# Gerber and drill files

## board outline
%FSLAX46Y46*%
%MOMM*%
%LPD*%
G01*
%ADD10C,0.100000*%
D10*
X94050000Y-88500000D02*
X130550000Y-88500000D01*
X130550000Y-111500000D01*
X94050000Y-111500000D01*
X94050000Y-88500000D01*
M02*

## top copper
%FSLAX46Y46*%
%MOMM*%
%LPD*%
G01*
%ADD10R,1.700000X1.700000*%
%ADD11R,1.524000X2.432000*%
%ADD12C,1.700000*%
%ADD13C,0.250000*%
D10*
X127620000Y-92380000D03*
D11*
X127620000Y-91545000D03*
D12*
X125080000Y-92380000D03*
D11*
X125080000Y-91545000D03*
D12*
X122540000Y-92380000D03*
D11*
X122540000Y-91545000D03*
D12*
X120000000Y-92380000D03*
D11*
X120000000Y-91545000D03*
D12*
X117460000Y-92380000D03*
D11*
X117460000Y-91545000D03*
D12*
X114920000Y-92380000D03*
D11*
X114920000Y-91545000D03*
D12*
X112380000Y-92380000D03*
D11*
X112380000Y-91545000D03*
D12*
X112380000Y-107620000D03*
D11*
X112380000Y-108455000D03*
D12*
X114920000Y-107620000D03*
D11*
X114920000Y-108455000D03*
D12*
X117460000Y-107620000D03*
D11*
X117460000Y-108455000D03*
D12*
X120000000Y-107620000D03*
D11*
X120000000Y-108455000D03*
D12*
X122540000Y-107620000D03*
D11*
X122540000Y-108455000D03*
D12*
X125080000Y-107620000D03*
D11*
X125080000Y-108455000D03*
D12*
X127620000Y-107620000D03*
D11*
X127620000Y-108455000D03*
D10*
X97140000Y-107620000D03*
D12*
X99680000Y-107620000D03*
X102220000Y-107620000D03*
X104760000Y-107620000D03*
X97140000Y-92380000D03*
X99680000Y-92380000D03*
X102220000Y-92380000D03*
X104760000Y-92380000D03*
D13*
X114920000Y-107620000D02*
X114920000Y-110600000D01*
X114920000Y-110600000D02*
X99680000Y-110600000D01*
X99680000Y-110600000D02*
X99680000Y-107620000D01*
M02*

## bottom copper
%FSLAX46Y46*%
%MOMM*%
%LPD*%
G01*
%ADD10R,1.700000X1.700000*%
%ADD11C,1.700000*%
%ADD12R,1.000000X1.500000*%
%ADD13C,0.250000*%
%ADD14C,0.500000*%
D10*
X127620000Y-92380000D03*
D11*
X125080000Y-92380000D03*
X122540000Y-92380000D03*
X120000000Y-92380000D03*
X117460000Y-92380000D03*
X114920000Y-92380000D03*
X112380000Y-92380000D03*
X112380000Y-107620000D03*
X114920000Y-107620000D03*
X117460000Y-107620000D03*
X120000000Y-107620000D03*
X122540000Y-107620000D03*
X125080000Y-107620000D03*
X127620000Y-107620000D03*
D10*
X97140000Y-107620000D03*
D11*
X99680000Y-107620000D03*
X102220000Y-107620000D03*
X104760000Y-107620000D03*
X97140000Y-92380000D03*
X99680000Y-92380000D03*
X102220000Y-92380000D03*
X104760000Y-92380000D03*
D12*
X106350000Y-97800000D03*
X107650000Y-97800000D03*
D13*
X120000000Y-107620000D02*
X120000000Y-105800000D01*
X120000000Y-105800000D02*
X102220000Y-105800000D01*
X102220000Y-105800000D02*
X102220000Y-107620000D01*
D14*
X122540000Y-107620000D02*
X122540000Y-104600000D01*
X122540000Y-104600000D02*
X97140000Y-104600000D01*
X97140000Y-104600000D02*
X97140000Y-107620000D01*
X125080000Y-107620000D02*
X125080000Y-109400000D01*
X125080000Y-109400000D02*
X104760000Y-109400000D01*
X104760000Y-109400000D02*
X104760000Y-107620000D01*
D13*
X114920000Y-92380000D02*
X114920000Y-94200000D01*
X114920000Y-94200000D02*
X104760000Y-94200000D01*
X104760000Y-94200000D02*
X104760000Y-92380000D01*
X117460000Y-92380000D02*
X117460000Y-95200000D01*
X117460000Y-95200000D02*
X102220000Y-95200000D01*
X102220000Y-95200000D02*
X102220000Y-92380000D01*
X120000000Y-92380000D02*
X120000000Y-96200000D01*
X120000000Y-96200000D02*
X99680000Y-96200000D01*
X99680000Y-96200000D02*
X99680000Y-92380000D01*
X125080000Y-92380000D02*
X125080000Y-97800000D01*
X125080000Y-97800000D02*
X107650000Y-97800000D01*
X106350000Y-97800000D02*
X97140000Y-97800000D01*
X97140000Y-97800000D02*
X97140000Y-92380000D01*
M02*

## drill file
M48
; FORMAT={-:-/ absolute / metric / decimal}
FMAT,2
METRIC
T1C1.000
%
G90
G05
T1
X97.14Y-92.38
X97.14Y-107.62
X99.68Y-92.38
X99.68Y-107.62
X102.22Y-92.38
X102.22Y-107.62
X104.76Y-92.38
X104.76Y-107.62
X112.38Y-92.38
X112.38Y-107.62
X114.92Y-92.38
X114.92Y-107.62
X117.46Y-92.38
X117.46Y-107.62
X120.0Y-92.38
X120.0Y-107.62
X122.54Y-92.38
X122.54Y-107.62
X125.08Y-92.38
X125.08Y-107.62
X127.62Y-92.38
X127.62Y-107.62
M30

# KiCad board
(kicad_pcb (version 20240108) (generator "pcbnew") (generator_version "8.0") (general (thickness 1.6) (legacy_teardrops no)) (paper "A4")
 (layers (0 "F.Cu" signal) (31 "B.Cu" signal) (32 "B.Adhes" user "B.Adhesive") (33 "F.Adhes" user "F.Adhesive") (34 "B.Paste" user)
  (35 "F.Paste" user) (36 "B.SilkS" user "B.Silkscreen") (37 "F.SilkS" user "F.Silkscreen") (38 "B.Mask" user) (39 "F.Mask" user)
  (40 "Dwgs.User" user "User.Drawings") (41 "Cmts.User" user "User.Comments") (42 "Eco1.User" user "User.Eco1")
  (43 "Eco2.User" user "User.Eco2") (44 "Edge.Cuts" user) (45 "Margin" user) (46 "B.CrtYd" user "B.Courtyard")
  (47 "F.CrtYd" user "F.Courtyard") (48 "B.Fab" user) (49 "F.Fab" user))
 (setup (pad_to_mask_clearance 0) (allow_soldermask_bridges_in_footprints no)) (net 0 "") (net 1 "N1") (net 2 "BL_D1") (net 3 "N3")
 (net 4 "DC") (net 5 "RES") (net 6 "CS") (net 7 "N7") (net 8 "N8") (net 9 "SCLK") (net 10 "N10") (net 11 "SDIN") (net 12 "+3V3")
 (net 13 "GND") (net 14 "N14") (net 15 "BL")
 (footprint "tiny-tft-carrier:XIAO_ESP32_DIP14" (layer "F.Cu") (at 120 100)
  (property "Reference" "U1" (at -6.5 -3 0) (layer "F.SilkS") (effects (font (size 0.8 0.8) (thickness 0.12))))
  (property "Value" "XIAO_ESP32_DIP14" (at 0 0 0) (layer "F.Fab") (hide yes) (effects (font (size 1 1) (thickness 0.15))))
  (pad "1" thru_hole rect (at 7.62 -7.62) (size 1.7 1.7) (drill 1) (layers "*.Cu" "*.Mask") (remove_unused_layers no) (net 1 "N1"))
  (pad "1" smd rect (at 7.62 -8.455) (size 1.524 2.432) (layers "F.Cu" "F.Mask") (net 1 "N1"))
  (pad "2" thru_hole circle (at 5.08 -7.62) (size 1.7 1.7) (drill 1) (layers "*.Cu" "*.Mask") (remove_unused_layers no) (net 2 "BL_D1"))
  (pad "2" smd rect (at 5.08 -8.455) (size 1.524 2.432) (layers "F.Cu" "F.Mask") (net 2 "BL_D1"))
  (pad "3" thru_hole circle (at 2.54 -7.62) (size 1.7 1.7) (drill 1) (layers "*.Cu" "*.Mask") (remove_unused_layers no) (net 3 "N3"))
  (pad "3" smd rect (at 2.54 -8.455) (size 1.524 2.432) (layers "F.Cu" "F.Mask") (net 3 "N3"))
  (pad "4" thru_hole circle (at 0 -7.62) (size 1.7 1.7) (drill 1) (layers "*.Cu" "*.Mask") (remove_unused_layers no) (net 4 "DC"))
  (pad "4" smd rect (at 0 -8.455) (size 1.524 2.432) (layers "F.Cu" "F.Mask") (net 4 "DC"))
  (pad "5" thru_hole circle (at -2.54 -7.62) (size 1.7 1.7) (drill 1) (layers "*.Cu" "*.Mask") (remove_unused_layers no) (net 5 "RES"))
  (pad "5" smd rect (at -2.54 -8.455) (size 1.524 2.432) (layers "F.Cu" "F.Mask") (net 5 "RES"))
  (pad "6" thru_hole circle (at -5.08 -7.62) (size 1.7 1.7) (drill 1) (layers "*.Cu" "*.Mask") (remove_unused_layers no) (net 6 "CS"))
  (pad "6" smd rect (at -5.08 -8.455) (size 1.524 2.432) (layers "F.Cu" "F.Mask") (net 6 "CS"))
  (pad "7" thru_hole circle (at -7.62 -7.62) (size 1.7 1.7) (drill 1) (layers "*.Cu" "*.Mask") (remove_unused_layers no) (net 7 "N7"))
  (pad "7" smd rect (at -7.62 -8.455) (size 1.524 2.432) (layers "F.Cu" "F.Mask") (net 7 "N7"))
  (pad "8" thru_hole circle (at -7.62 7.62) (size 1.7 1.7) (drill 1) (layers "*.Cu" "*.Mask") (remove_unused_layers no) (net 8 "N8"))
  (pad "8" smd rect (at -7.62 8.455) (size 1.524 2.432) (layers "F.Cu" "F.Mask") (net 8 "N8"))
  (pad "9" thru_hole circle (at -5.08 7.62) (size 1.7 1.7) (drill 1) (layers "*.Cu" "*.Mask") (remove_unused_layers no) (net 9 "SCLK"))
  (pad "9" smd rect (at -5.08 8.455) (size 1.524 2.432) (layers "F.Cu" "F.Mask") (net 9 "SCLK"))
  (pad "10" thru_hole circle (at -2.54 7.62) (size 1.7 1.7) (drill 1) (layers "*.Cu" "*.Mask") (remove_unused_layers no) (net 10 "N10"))
  (pad "10" smd rect (at -2.54 8.455) (size 1.524 2.432) (layers "F.Cu" "F.Mask") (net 10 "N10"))
  (pad "11" thru_hole circle (at 0 7.62) (size 1.7 1.7) (drill 1) (layers "*.Cu" "*.Mask") (remove_unused_layers no) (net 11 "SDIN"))
  (pad "11" smd rect (at 0 8.455) (size 1.524 2.432) (layers "F.Cu" "F.Mask") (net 11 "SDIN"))
  (pad "12" thru_hole circle (at 2.54 7.62) (size 1.7 1.7) (drill 1) (layers "*.Cu" "*.Mask") (remove_unused_layers no) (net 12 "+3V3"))
  (pad "12" smd rect (at 2.54 8.455) (size 1.524 2.432) (layers "F.Cu" "F.Mask") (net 12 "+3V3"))
  (pad "13" thru_hole circle (at 5.08 7.62) (size 1.7 1.7) (drill 1) (layers "*.Cu" "*.Mask") (remove_unused_layers no) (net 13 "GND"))
  (pad "13" smd rect (at 5.08 8.455) (size 1.524 2.432) (layers "F.Cu" "F.Mask") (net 13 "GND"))
  (pad "14" thru_hole circle (at 7.62 7.62) (size 1.7 1.7) (drill 1) (layers "*.Cu" "*.Mask") (remove_unused_layers no) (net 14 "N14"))
  (pad "14" smd rect (at 7.62 8.455) (size 1.524 2.432) (layers "F.Cu" "F.Mask") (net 14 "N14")))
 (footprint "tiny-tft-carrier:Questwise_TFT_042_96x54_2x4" (layer "F.Cu") (at 100.95 100)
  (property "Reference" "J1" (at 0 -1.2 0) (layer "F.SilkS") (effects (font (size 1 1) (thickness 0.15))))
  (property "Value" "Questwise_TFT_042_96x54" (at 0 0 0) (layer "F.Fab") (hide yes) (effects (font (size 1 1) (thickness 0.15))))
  (pad "1" thru_hole rect (at -3.81 7.62) (size 1.7 1.7) (drill 1) (layers "*.Cu" "*.Mask") (remove_unused_layers no) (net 12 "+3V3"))
  (pad "2" thru_hole circle (at -1.27 7.62) (size 1.7 1.7) (drill 1) (layers "*.Cu" "*.Mask") (remove_unused_layers no) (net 9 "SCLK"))
  (pad "3" thru_hole circle (at 1.27 7.62) (size 1.7 1.7) (drill 1) (layers "*.Cu" "*.Mask") (remove_unused_layers no) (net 11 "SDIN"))
  (pad "4" thru_hole circle (at 3.81 7.62) (size 1.7 1.7) (drill 1) (layers "*.Cu" "*.Mask") (remove_unused_layers no) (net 13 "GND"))
  (pad "5" thru_hole circle (at -3.81 -7.62) (size 1.7 1.7) (drill 1) (layers "*.Cu" "*.Mask") (remove_unused_layers no) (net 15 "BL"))
  (pad "6" thru_hole circle (at -1.27 -7.62) (size 1.7 1.7) (drill 1) (layers "*.Cu" "*.Mask") (remove_unused_layers no) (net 4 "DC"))
  (pad "7" thru_hole circle (at 1.27 -7.62) (size 1.7 1.7) (drill 1) (layers "*.Cu" "*.Mask") (remove_unused_layers no) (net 5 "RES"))
  (pad "8" thru_hole circle (at 3.81 -7.62) (size 1.7 1.7) (drill 1) (layers "*.Cu" "*.Mask") (remove_unused_layers no) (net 6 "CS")))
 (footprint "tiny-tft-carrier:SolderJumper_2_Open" (layer "B.Cu") (at 107 97.8)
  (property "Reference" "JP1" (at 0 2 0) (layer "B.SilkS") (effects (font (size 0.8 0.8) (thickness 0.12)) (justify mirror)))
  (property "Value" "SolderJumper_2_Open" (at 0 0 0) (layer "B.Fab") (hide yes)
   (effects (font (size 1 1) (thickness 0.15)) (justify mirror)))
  (pad "1" smd rect (at -0.65 0) (size 1 1.5) (layers "B.Cu" "B.Mask") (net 15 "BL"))
  (pad "2" smd rect (at 0.65 0) (size 1 1.5) (layers "B.Cu" "B.Mask") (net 2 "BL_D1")))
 (gr_rect (start 94.05 88.5) (end 130.55 111.5) (stroke (width 0.1) (type default)) (fill no) (layer "Edge.Cuts"))
 (segment (start 120 107.62) (end 120 105.8) (width 0.25) (layer "B.Cu") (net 11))
 (segment (start 120 105.8) (end 102.22 105.8) (width 0.25) (layer "B.Cu") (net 11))
 (segment (start 102.22 105.8) (end 102.22 107.62) (width 0.25) (layer "B.Cu") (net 11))
 (segment (start 122.54 107.62) (end 122.54 104.6) (width 0.5) (layer "B.Cu") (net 12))
 (segment (start 122.54 104.6) (end 97.14 104.6) (width 0.5) (layer "B.Cu") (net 12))
 (segment (start 97.14 104.6) (end 97.14 107.62) (width 0.5) (layer "B.Cu") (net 12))
 (segment (start 125.08 107.62) (end 125.08 109.4) (width 0.5) (layer "B.Cu") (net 13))
 (segment (start 125.08 109.4) (end 104.76 109.4) (width 0.5) (layer "B.Cu") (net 13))
 (segment (start 104.76 109.4) (end 104.76 107.62) (width 0.5) (layer "B.Cu") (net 13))
 (segment (start 114.92 107.62) (end 114.92 110.6) (width 0.25) (layer "F.Cu") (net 9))
 (segment (start 114.92 110.6) (end 99.68 110.6) (width 0.25) (layer "F.Cu") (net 9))
 (segment (start 99.68 110.6) (end 99.68 107.62) (width 0.25) (layer "F.Cu") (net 9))
 (segment (start 114.92 92.38) (end 114.92 94.2) (width 0.25) (layer "B.Cu") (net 6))
 (segment (start 114.92 94.2) (end 104.76 94.2) (width 0.25) (layer "B.Cu") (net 6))
 (segment (start 104.76 94.2) (end 104.76 92.38) (width 0.25) (layer "B.Cu") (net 6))
 (segment (start 117.46 92.38) (end 117.46 95.2) (width 0.25) (layer "B.Cu") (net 5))
 (segment (start 117.46 95.2) (end 102.22 95.2) (width 0.25) (layer "B.Cu") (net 5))
 (segment (start 102.22 95.2) (end 102.22 92.38) (width 0.25) (layer "B.Cu") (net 5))
 (segment (start 120 92.38) (end 120 96.2) (width 0.25) (layer "B.Cu") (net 4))
 (segment (start 120 96.2) (end 99.68 96.2) (width 0.25) (layer "B.Cu") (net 4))
 (segment (start 99.68 96.2) (end 99.68 92.38) (width 0.25) (layer "B.Cu") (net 4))
 (segment (start 125.08 92.38) (end 125.08 97.8) (width 0.25) (layer "B.Cu") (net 2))
 (segment (start 125.08 97.8) (end 107.65 97.8) (width 0.25) (layer "B.Cu") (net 2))
 (segment (start 106.35 97.8) (end 97.14 97.8) (width 0.25) (layer "B.Cu") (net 15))
 (segment (start 97.14 97.8) (end 97.14 92.38) (width 0.25) (layer "B.Cu") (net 15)))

